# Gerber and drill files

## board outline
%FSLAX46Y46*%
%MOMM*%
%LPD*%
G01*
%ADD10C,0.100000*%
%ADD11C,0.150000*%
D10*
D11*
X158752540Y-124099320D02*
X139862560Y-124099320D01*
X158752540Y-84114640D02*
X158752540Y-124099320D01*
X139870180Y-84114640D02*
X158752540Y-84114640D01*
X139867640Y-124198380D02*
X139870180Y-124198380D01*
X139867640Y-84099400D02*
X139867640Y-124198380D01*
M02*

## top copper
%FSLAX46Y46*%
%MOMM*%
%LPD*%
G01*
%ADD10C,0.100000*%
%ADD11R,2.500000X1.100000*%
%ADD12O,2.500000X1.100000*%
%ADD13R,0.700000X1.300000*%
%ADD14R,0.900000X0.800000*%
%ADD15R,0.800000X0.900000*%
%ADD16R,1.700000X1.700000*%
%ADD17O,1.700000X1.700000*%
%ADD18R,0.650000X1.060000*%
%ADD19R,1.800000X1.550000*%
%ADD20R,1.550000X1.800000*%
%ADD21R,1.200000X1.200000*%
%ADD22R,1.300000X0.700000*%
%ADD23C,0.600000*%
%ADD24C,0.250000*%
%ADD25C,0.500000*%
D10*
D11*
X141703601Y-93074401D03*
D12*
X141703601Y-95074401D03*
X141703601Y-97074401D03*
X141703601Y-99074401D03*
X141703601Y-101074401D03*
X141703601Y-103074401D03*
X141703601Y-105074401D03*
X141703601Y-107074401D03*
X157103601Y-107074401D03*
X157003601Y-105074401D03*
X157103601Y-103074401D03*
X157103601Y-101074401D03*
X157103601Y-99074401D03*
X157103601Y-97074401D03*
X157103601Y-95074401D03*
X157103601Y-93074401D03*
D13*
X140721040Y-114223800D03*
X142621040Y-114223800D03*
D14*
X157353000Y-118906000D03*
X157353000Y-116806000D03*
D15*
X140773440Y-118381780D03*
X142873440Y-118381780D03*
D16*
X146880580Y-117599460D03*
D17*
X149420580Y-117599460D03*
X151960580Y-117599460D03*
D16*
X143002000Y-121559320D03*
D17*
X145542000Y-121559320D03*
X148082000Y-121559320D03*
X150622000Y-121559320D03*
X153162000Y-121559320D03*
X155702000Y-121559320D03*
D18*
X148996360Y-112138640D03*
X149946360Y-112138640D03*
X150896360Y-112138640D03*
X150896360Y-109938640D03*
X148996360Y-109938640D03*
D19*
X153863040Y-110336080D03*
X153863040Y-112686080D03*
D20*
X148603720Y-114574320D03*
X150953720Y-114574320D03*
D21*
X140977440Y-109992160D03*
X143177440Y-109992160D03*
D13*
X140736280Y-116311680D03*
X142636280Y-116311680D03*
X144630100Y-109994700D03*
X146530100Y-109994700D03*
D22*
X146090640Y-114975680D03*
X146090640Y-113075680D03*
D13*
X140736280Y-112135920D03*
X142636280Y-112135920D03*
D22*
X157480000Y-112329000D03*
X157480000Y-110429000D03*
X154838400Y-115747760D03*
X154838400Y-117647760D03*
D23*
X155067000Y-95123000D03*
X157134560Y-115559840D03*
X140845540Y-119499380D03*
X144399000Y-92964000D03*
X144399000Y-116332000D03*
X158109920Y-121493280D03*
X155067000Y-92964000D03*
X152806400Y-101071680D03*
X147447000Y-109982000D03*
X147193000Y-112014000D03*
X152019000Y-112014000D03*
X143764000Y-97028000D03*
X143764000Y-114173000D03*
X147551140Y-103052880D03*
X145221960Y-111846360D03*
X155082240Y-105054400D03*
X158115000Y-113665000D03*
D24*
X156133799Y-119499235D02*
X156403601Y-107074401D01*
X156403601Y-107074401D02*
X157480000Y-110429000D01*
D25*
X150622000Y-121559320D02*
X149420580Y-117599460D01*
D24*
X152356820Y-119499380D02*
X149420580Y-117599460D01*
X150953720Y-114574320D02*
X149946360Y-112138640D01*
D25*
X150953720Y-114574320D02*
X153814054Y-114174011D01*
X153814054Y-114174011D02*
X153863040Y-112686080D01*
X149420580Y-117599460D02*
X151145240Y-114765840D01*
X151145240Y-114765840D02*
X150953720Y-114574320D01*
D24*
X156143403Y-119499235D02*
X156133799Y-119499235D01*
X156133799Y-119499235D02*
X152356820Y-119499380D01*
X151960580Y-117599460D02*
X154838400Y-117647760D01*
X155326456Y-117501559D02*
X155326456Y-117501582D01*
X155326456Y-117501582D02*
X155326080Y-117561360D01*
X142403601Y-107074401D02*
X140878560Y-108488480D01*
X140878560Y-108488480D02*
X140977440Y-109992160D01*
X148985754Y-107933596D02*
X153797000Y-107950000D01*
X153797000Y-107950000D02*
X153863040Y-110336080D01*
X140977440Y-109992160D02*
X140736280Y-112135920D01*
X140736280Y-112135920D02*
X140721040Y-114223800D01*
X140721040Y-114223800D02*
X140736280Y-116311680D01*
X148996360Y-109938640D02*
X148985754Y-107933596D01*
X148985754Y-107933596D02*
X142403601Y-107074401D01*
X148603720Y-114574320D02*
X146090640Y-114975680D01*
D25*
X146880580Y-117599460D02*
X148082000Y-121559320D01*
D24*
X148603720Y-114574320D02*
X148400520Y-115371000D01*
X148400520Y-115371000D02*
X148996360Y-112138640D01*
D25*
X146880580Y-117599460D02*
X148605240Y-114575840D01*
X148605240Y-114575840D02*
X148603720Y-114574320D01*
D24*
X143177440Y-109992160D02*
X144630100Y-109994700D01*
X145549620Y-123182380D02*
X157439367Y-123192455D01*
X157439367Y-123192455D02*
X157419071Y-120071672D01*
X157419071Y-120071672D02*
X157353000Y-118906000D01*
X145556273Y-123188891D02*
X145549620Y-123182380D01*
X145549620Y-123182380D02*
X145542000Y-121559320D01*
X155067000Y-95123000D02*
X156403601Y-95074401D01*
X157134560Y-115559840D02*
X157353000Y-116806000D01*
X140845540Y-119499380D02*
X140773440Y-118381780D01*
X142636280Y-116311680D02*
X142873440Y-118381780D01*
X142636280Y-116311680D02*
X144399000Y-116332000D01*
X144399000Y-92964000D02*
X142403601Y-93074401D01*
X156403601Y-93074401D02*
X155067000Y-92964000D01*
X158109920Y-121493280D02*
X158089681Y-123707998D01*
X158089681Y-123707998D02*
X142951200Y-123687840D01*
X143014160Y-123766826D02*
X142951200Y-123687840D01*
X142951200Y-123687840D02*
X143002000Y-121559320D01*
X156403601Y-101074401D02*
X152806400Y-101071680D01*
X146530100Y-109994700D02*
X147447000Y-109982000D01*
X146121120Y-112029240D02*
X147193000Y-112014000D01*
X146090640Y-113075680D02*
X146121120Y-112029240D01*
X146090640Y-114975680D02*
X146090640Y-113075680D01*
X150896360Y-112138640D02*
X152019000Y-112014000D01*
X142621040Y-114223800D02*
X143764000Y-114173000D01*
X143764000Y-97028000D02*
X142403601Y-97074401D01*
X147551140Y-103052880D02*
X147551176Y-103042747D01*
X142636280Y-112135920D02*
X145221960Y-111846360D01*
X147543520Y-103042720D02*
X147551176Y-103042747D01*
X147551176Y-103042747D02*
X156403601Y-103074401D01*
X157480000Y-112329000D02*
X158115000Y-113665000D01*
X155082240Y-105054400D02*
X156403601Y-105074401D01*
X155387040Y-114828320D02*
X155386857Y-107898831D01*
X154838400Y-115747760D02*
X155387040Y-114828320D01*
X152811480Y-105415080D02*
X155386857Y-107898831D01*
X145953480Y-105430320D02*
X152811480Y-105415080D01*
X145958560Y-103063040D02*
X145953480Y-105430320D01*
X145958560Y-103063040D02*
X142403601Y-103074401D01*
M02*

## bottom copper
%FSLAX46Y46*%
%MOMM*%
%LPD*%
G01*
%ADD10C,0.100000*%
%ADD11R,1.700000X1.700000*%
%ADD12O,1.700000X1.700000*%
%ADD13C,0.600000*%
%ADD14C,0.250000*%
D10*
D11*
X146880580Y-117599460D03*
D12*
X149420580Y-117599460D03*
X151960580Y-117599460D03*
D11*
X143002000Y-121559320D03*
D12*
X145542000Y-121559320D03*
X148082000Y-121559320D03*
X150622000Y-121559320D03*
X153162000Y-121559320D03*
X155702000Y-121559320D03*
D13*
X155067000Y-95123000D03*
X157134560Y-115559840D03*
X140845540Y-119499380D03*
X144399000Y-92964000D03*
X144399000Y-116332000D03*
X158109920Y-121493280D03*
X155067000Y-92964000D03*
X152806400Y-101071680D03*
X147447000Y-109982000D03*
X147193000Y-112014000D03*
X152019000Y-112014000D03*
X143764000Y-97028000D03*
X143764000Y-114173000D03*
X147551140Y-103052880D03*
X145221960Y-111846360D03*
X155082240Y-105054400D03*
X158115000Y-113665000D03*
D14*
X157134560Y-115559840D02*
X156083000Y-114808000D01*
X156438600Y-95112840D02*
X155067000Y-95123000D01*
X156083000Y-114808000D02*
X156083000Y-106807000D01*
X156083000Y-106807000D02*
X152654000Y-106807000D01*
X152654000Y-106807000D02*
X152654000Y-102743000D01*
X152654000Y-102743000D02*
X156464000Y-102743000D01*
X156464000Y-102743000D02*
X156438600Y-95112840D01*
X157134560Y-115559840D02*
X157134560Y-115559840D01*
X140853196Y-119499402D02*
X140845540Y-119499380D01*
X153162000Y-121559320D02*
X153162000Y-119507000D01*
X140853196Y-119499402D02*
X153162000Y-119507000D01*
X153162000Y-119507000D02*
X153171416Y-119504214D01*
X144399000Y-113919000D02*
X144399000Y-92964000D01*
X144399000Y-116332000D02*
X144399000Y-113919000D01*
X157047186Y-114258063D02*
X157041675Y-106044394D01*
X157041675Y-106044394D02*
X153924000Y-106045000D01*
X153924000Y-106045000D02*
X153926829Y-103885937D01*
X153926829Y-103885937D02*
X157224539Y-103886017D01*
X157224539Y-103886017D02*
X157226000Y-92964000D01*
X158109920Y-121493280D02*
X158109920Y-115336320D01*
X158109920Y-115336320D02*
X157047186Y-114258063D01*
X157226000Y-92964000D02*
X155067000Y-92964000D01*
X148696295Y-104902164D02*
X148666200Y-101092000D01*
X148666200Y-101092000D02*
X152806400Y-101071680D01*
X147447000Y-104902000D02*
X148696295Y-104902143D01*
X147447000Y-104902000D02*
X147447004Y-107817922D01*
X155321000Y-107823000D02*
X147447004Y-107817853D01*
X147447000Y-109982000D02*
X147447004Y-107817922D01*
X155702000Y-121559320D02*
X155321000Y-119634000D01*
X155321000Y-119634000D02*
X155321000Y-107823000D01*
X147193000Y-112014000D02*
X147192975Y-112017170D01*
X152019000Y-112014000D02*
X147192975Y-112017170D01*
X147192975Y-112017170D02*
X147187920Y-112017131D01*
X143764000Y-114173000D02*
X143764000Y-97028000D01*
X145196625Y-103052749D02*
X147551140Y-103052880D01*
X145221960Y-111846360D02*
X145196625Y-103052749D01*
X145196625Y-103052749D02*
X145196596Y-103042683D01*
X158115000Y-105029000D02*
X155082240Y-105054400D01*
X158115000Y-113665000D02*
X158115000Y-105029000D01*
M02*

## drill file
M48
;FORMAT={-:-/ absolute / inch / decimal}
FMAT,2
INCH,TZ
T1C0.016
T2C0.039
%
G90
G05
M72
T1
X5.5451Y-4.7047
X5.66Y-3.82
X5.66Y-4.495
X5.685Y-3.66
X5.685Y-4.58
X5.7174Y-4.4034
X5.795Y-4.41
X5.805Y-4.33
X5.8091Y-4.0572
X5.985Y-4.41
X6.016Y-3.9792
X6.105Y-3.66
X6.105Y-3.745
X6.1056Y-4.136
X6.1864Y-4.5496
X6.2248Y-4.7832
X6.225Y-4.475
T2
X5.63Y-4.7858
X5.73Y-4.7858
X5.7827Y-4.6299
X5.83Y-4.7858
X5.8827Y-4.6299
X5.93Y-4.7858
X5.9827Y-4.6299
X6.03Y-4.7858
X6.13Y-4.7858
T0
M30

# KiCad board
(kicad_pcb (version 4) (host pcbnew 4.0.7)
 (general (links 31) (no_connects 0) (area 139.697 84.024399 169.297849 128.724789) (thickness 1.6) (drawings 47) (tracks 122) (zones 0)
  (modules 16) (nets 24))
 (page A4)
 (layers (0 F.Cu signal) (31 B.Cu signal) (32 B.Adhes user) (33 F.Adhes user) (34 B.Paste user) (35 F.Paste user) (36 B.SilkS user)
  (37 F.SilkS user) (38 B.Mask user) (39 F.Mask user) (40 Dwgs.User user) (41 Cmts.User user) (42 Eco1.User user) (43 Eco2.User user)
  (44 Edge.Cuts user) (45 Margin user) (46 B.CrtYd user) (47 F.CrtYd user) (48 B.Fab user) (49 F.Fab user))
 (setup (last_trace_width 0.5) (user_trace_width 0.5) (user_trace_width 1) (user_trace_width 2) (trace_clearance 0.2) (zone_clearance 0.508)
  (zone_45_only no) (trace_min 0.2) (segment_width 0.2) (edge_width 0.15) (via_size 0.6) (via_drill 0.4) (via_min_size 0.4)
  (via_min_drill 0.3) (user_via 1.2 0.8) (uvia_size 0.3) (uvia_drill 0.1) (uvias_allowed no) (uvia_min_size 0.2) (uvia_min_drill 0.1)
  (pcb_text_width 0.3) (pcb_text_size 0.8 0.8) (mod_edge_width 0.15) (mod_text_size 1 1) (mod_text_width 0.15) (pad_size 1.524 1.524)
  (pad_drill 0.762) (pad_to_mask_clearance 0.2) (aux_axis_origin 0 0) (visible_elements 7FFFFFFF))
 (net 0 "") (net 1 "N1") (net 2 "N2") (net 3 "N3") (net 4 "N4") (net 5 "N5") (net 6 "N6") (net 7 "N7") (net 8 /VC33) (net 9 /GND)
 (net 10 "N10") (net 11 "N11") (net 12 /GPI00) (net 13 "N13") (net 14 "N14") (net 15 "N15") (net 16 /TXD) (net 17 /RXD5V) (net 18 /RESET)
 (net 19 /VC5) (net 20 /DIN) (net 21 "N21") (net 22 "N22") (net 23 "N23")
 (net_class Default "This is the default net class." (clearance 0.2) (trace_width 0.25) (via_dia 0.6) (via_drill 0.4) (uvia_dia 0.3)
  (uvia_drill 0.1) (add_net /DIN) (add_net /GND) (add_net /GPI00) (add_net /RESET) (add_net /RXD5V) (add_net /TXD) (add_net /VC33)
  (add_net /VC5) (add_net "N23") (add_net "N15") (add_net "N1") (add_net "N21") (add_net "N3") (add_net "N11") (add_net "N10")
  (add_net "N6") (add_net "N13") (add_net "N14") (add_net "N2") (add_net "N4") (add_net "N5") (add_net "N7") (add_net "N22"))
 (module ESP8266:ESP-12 (layer F.Cu) (at 142.403601 93.074401)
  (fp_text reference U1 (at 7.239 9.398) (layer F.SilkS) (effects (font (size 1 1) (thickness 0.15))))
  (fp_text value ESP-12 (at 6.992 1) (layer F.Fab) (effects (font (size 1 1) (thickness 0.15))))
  (pad 1 smd rect (at 0 0) (size 2.5 1.1) (drill (offset -0.7 0)) (layers F.Cu F.Paste F.Mask) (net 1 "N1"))
  (pad 2 smd oval (at 0 2) (size 2.5 1.1) (drill (offset -0.7 0)) (layers F.Cu F.Paste F.Mask) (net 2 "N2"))
  (pad 3 smd oval (at 0 4) (size 2.5 1.1) (drill (offset -0.7 0)) (layers F.Cu F.Paste F.Mask) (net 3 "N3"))
  (pad 4 smd oval (at 0 6) (size 2.5 1.1) (drill (offset -0.7 0)) (layers F.Cu F.Paste F.Mask) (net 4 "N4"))
  (pad 5 smd oval (at 0 8) (size 2.5 1.1) (drill (offset -0.7 0)) (layers F.Cu F.Paste F.Mask) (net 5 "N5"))
  (pad 6 smd oval (at 0 10) (size 2.5 1.1) (drill (offset -0.7 0)) (layers F.Cu F.Paste F.Mask) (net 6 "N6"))
  (pad 7 smd oval (at 0 12) (size 2.5 1.1) (drill (offset -0.7 0)) (layers F.Cu F.Paste F.Mask) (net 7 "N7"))
  (pad 8 smd oval (at 0 14) (size 2.5 1.1) (drill (offset -0.7 0)) (layers F.Cu F.Paste F.Mask) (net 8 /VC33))
  (pad 9 smd oval (at 14 14) (size 2.5 1.1) (drill (offset 0.7 0)) (layers F.Cu F.Paste F.Mask) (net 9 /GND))
  (pad 10 smd oval (at 14 12) (size 2.5 1.1) (drill (offset 0.6 0)) (layers F.Cu F.Paste F.Mask) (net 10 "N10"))
  (pad 11 smd oval (at 14 10) (size 2.5 1.1) (drill (offset 0.7 0)) (layers F.Cu F.Paste F.Mask) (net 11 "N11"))
  (pad 12 smd oval (at 14 8) (size 2.5 1.1) (drill (offset 0.7 0)) (layers F.Cu F.Paste F.Mask) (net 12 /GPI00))
  (pad 13 smd oval (at 14 6) (size 2.5 1.1) (drill (offset 0.7 0)) (layers F.Cu F.Paste F.Mask) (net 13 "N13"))
  (pad 14 smd oval (at 14 4) (size 2.5 1.1) (drill (offset 0.7 0)) (layers F.Cu F.Paste F.Mask) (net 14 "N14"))
  (pad 15 smd oval (at 14 2) (size 2.5 1.1) (drill (offset 0.7 0)) (layers F.Cu F.Paste F.Mask) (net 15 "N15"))
  (pad 16 smd oval (at 14 0) (size 2.5 1.1) (drill (offset 0.7 0)) (layers F.Cu F.Paste F.Mask) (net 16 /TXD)))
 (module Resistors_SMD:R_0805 (layer F.Cu) (at 141.67104 114.2238)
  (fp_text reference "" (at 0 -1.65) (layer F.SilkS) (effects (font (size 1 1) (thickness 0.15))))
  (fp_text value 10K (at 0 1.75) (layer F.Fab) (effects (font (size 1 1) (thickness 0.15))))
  (pad 1 smd rect (at -0.95 0) (size 0.7 1.3) (layers F.Cu F.Paste F.Mask) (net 8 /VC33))
  (pad 2 smd rect (at 0.95 0) (size 0.7 1.3) (layers F.Cu F.Paste F.Mask) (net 3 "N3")))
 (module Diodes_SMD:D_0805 (layer F.Cu) (at 157.353 117.856 90)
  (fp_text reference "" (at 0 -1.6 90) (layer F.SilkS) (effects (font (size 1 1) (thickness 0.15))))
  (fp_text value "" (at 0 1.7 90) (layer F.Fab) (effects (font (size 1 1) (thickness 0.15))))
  (pad 1 smd rect (at -1.05 0 90) (size 0.8 0.9) (layers F.Cu F.Paste F.Mask) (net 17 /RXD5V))
  (pad 2 smd rect (at 1.05 0 90) (size 0.8 0.9) (layers F.Cu F.Paste F.Mask) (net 15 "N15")))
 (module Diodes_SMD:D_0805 (layer F.Cu) (at 141.82344 118.38178)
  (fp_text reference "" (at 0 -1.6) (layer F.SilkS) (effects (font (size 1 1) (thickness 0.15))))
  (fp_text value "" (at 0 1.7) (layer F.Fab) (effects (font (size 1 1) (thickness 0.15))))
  (pad 1 smd rect (at -1.05 0) (size 0.8 0.9) (layers F.Cu F.Paste F.Mask) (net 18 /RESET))
  (pad 2 smd rect (at 1.05 0) (size 0.8 0.9) (layers F.Cu F.Paste F.Mask) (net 1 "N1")))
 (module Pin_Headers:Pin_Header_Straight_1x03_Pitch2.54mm (layer F.Cu) (at 146.88058 117.59946 90)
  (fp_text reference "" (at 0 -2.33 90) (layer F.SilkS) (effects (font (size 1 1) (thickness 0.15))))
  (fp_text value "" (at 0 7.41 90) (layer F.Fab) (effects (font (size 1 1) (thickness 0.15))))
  (pad 1 thru_hole rect (at 0 0 90) (size 1.7 1.7) (drill 1) (layers *.Cu *.Mask) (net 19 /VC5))
  (pad 2 thru_hole oval (at 0 2.54 90) (size 1.7 1.7) (drill 1) (layers *.Cu *.Mask) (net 9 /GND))
  (pad 3 thru_hole oval (at 0 5.08 90) (size 1.7 1.7) (drill 1) (layers *.Cu *.Mask) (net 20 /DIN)))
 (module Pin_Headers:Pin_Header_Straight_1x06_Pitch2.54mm (layer F.Cu) (at 143.002 121.55932 90)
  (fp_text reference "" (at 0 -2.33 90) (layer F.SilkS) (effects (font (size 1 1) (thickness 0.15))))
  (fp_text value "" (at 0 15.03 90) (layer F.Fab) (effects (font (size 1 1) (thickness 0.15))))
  (pad 1 thru_hole rect (at 0 0 90) (size 1.7 1.7) (drill 1) (layers *.Cu *.Mask) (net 16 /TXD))
  (pad 2 thru_hole oval (at 0 2.54 90) (size 1.7 1.7) (drill 1) (layers *.Cu *.Mask) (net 17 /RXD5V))
  (pad 3 thru_hole oval (at 0 5.08 90) (size 1.7 1.7) (drill 1) (layers *.Cu *.Mask) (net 19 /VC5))
  (pad 4 thru_hole oval (at 0 7.62 90) (size 1.7 1.7) (drill 1) (layers *.Cu *.Mask) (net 9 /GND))
  (pad 5 thru_hole oval (at 0 10.16 90) (size 1.7 1.7) (drill 1) (layers *.Cu *.Mask) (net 18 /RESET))
  (pad 6 thru_hole oval (at 0 12.7 90) (size 1.7 1.7) (drill 1) (layers *.Cu *.Mask) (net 12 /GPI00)))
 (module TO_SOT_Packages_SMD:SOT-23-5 (layer F.Cu) (at 149.94636 111.03864 90)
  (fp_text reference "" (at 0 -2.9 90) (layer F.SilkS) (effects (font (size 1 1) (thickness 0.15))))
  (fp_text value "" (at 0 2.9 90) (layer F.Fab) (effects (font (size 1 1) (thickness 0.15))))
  (pad 1 smd rect (at -1.1 -0.95 90) (size 1.06 0.65) (layers F.Cu F.Paste F.Mask) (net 19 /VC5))
  (pad 2 smd rect (at -1.1 0 90) (size 1.06 0.65) (layers F.Cu F.Paste F.Mask) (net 9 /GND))
  (pad 3 smd rect (at -1.1 0.95 90) (size 1.06 0.65) (layers F.Cu F.Paste F.Mask) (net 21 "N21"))
  (pad 4 smd rect (at 1.1 0.95 90) (size 1.06 0.65) (layers F.Cu F.Paste F.Mask) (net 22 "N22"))
  (pad 5 smd rect (at 1.1 -0.95 90) (size 1.06 0.65) (layers F.Cu F.Paste F.Mask) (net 8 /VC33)))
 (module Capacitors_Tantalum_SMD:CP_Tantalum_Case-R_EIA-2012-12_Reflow (layer F.Cu) (at 153.86304 111.51108 270)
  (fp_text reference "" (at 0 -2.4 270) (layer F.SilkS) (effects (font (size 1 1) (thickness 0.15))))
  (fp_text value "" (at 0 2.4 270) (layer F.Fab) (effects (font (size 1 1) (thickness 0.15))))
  (pad 1 smd rect (at -1.175 0 270) (size 1.55 1.8) (layers F.Cu F.Paste F.Mask) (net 8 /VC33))
  (pad 2 smd rect (at 1.175 0 270) (size 1.55 1.8) (layers F.Cu F.Paste F.Mask) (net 9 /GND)))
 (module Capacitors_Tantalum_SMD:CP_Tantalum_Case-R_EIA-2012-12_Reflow (layer F.Cu) (at 149.77872 114.57432)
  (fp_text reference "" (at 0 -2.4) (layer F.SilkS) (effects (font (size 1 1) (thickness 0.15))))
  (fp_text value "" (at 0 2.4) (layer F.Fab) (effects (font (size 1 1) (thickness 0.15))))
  (pad 1 smd rect (at -1.175 0) (size 1.55 1.8) (layers F.Cu F.Paste F.Mask) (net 19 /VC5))
  (pad 2 smd rect (at 1.175 0) (size 1.55 1.8) (layers F.Cu F.Paste F.Mask) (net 9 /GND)))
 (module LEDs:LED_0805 (layer F.Cu) (at 142.07744 109.99216 180)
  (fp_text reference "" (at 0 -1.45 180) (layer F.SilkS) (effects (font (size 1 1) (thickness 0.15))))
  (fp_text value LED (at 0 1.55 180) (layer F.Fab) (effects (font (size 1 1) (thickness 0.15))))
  (pad 2 smd rect (at 1.1 0) (size 1.2 1.2) (layers F.Cu F.Paste F.Mask) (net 8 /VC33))
  (pad 1 smd rect (at -1.1 0) (size 1.2 1.2) (layers F.Cu F.Paste F.Mask) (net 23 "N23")))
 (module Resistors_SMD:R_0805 (layer F.Cu) (at 141.68628 116.31168)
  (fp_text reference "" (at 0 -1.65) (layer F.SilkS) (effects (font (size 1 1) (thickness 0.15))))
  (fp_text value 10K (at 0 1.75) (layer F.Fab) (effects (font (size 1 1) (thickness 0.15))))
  (pad 1 smd rect (at -0.95 0) (size 0.7 1.3) (layers F.Cu F.Paste F.Mask) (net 8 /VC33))
  (pad 2 smd rect (at 0.95 0) (size 0.7 1.3) (layers F.Cu F.Paste F.Mask) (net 1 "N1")))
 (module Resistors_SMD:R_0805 (layer F.Cu) (at 145.5801 109.9947)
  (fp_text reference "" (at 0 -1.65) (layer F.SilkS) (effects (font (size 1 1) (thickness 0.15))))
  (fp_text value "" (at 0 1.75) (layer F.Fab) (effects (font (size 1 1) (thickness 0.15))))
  (pad 1 smd rect (at -0.95 0) (size 0.7 1.3) (layers F.Cu F.Paste F.Mask) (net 23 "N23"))
  (pad 2 smd rect (at 0.95 0) (size 0.7 1.3) (layers F.Cu F.Paste F.Mask) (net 12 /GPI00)))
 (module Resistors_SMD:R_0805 (layer F.Cu) (at 146.09064 114.02568 90)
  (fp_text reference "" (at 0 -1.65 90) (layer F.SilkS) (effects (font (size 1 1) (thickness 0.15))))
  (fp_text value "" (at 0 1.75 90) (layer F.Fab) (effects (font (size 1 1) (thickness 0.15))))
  (pad 1 smd rect (at -0.95 0 90) (size 0.7 1.3) (layers F.Cu F.Paste F.Mask) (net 19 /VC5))
  (pad 2 smd rect (at 0.95 0 90) (size 0.7 1.3) (layers F.Cu F.Paste F.Mask) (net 21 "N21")))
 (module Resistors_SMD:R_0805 (layer F.Cu) (at 141.68628 112.13592)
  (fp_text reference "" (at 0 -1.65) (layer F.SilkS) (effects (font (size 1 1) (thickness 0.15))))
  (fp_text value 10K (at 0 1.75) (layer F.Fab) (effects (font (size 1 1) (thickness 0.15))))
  (pad 1 smd rect (at -0.95 0) (size 0.7 1.3) (layers F.Cu F.Paste F.Mask) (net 8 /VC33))
  (pad 2 smd rect (at 0.95 0) (size 0.7 1.3) (layers F.Cu F.Paste F.Mask) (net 11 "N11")))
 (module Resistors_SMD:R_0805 (layer F.Cu) (at 157.48 111.379 90)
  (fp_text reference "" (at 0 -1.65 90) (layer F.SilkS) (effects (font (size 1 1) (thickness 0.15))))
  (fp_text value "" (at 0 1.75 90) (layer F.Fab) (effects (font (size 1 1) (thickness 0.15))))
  (pad 1 smd rect (at -0.95 0 90) (size 0.7 1.3) (layers F.Cu F.Paste F.Mask) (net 10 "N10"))
  (pad 2 smd rect (at 0.95 0 90) (size 0.7 1.3) (layers F.Cu F.Paste F.Mask) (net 9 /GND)))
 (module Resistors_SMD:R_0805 (layer F.Cu) (at 154.8384 116.69776 270)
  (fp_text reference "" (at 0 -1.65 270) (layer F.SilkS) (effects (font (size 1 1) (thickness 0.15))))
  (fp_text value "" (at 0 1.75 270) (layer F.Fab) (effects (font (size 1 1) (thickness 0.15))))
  (pad 1 smd rect (at -0.95 0 270) (size 0.7 1.3) (layers F.Cu F.Paste F.Mask) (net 6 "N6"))
  (pad 2 smd rect (at 0.95 0 270) (size 0.7 1.3) (layers F.Cu F.Paste F.Mask) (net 20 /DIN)))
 (gr_line (start 158.75254 124.09932) (end 139.86256 124.09932) (angle 90) (layer Edge.Cuts) (width 0.15))
 (gr_line (start 158.75254 84.11464) (end 158.75254 124.09932) (angle 90) (layer Edge.Cuts) (width 0.15))
 (gr_line (start 139.87018 84.11464) (end 158.75254 84.11464) (angle 90) (layer Edge.Cuts) (width 0.15))
 (gr_line (start 139.86764 124.19838) (end 139.87018 124.19838) (angle 90) (layer Edge.Cuts) (width 0.15))
 (gr_line (start 139.86764 84.0994) (end 139.86764 124.19838) (angle 90) (layer Edge.Cuts) (width 0.15))
 (segment (start 156.133799 119.499235) (end 156.403601 107.074401) (width 0.25) (layer F.Cu) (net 9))
 (segment (start 156.403601 107.074401) (end 157.48 110.429) (width 0.25) (layer F.Cu) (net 9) (status 20))
 (segment (start 150.622 121.55932) (end 149.42058 117.59946) (width 0.5) (layer F.Cu) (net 9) (status 20))
 (segment (start 152.35682 119.49938) (end 149.42058 117.59946) (width 0.25) (layer F.Cu) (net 9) (status 20))
 (segment (start 150.95372 114.57432) (end 149.94636 112.13864) (width 0.25) (layer F.Cu) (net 9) (status 10))
 (segment (start 150.95372 114.57432) (end 153.814054 114.174011) (width 0.5) (layer F.Cu) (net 9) (status 10))
 (segment (start 153.814054 114.174011) (end 153.86304 112.68608) (width 0.5) (layer F.Cu) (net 9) (status 10))
 (segment (start 149.42058 117.59946) (end 151.14524 114.76584) (width 0.5) (layer F.Cu) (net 9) (status 20))
 (segment (start 151.14524 114.76584) (end 150.95372 114.57432) (width 0.5) (layer F.Cu) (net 9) (status 30))
 (segment (start 156.143403 119.499235) (end 156.133799 119.499235) (width 0.25) (layer F.Cu) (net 9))
 (segment (start 156.133799 119.499235) (end 152.35682 119.49938) (width 0.25) (layer F.Cu) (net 9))
 (segment (start 151.96058 117.59946) (end 154.8384 117.64776) (width 0.25) (layer F.Cu) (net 20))
 (segment (start 155.326456 117.501559) (end 155.326456 117.501582) (width 0.25) (layer F.Cu) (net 20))
 (segment (start 155.326456 117.501582) (end 155.32608 117.56136) (width 0.25) (layer F.Cu) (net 20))
 (segment (start 142.403601 107.074401) (end 140.87856 108.48848) (width 0.25) (layer F.Cu) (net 8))
 (segment (start 140.87856 108.48848) (end 140.97744 109.99216) (width 0.25) (layer F.Cu) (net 8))
 (segment (start 148.985754 107.933596) (end 153.797 107.95) (width 0.25) (layer F.Cu) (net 8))
 (segment (start 153.797 107.95) (end 153.86304 110.33608) (width 0.25) (layer F.Cu) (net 8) (status 20))
 (segment (start 140.97744 109.99216) (end 140.73628 112.13592) (width 0.25) (layer F.Cu) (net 8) (status 20))
 (segment (start 140.73628 112.13592) (end 140.72104 114.2238) (width 0.25) (layer F.Cu) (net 8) (status 20))
 (segment (start 140.72104 114.2238) (end 140.73628 116.31168) (width 0.25) (layer F.Cu) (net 8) (status 20))
 (segment (start 148.99636 109.93864) (end 148.985754 107.933596) (width 0.25) (layer F.Cu) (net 8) (status 10))
 (segment (start 148.985754 107.933596) (end 142.403601 107.074401) (width 0.25) (layer F.Cu) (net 8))
 (segment (start 148.60372 114.57432) (end 146.09064 114.97568) (width 0.25) (layer F.Cu) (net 19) (status 10))
 (segment (start 146.88058 117.59946) (end 148.082 121.55932) (width 0.5) (layer F.Cu) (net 19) (status 10))
 (segment (start 148.60372 114.57432) (end 148.40052 115.371) (width 0.25) (layer F.Cu) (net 19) (status 30))
 (segment (start 148.40052 115.371) (end 148.99636 112.13864) (width 0.25) (layer F.Cu) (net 19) (status 10))
 (segment (start 146.88058 117.59946) (end 148.60524 114.57584) (width 0.5) (layer F.Cu) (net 19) (status 20))
 (segment (start 148.60524 114.57584) (end 148.60372 114.57432) (width 0.5) (layer F.Cu) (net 19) (status 30))
 (segment (start 143.17744 109.99216) (end 144.6301 109.9947) (width 0.25) (layer F.Cu) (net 23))
 (segment (start 145.54962 123.18238) (end 157.439367 123.192455) (width 0.25) (layer F.Cu) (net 17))
 (segment (start 157.439367 123.192455) (end 157.419071 120.071672) (width 0.25) (layer F.Cu) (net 17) (status 20))
 (segment (start 157.419071 120.071672) (end 157.353 118.906) (width 0.25) (layer F.Cu) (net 17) (status 20))
 (segment (start 145.556273 123.188891) (end 145.54962 123.18238) (width 0.25) (layer F.Cu) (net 17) (status 20))
 (segment (start 145.54962 123.18238) (end 145.542 121.55932) (width 0.25) (layer F.Cu) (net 17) (status 20))
 (segment (start 157.13456 115.55984) (end 156.083 114.808) (width 0.25) (layer B.Cu) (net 15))
 (via (at 155.067 95.123) (size 0.6) (drill 0.4) (layers F.Cu B.Cu) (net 15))
 (segment (start 155.067 95.123) (end 156.403601 95.074401) (width 0.25) (layer F.Cu) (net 15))
 (segment (start 156.4386 95.11284) (end 155.067 95.123) (width 0.25) (layer B.Cu) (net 15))
 (segment (start 156.083 114.808) (end 156.083 106.807) (width 0.25) (layer B.Cu) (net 15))
 (segment (start 156.083 106.807) (end 152.654 106.807) (width 0.25) (layer B.Cu) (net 15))
 (segment (start 152.654 106.807) (end 152.654 102.743) (width 0.25) (layer B.Cu) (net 15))
 (segment (start 152.654 102.743) (end 156.464 102.743) (width 0.25) (layer B.Cu) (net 15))
 (segment (start 156.464 102.743) (end 156.4386 95.11284) (width 0.25) (layer B.Cu) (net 15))
 (segment (start 157.13456 115.55984) (end 157.353 116.806) (width 0.25) (layer F.Cu) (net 15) (status 20))
 (via (at 157.13456 115.55984) (size 0.6) (drill 0.4) (layers F.Cu B.Cu) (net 15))
 (segment (start 157.13456 115.55984) (end 157.13456 115.55984) (width 0.25) (layer B.Cu) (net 15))
 (segment (start 140.853196 119.499402) (end 140.84554 119.49938) (width 0.25) (layer B.Cu) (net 18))
 (via (at 140.84554 119.49938) (size 0.6) (drill 0.4) (layers F.Cu B.Cu) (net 18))
 (segment (start 140.84554 119.49938) (end 140.77344 118.38178) (width 0.25) (layer F.Cu) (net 18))
 (segment (start 153.162 121.55932) (end 153.162 119.507) (width 0.25) (layer B.Cu) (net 18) (status 10))
 (segment (start 140.853196 119.499402) (end 153.162 119.507) (width 0.25) (layer B.Cu) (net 18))
 (segment (start 153.162 119.507) (end 153.171416 119.504214) (width 0.25) (layer B.Cu) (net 18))
 (segment (start 142.63628 116.31168) (end 142.87344 118.38178) (width 0.25) (layer F.Cu) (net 1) (status 10))
 (segment (start 142.63628 116.31168) (end 144.399 116.332) (width 0.25) (layer F.Cu) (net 1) (status 10))
 (segment (start 144.399 92.964) (end 142.403601 93.074401) (width 0.25) (layer F.Cu) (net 1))
 (via (at 144.399 92.964) (size 0.6) (drill 0.4) (layers F.Cu B.Cu) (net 1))
 (segment (start 144.399 113.919) (end 144.399 92.964) (width 0.25) (layer B.Cu) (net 1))
 (segment (start 144.399 116.332) (end 144.399 113.919) (width 0.25) (layer B.Cu) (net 1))
 (via (at 144.399 116.332) (size 0.6) (drill 0.4) (layers F.Cu B.Cu) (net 1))
 (segment (start 157.047186 114.258063) (end 157.041675 106.044394) (width 0.25) (layer B.Cu) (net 16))
 (segment (start 157.041675 106.044394) (end 153.924 106.045) (width 0.25) (layer B.Cu) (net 16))
 (segment (start 153.924 106.045) (end 153.926829 103.885937) (width 0.25) (layer B.Cu) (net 16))
 (segment (start 153.926829 103.885937) (end 157.224539 103.886017) (width 0.25) (layer B.Cu) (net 16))
 (segment (start 157.224539 103.886017) (end 157.226 92.964) (width 0.25) (layer B.Cu) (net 16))
 (via (at 158.10992 121.49328) (size 0.6) (drill 0.4) (layers F.Cu B.Cu) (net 16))
 (segment (start 158.10992 121.49328) (end 158.10992 115.33632) (width 0.25) (layer B.Cu) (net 16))
 (via (at 155.067 92.964) (size 0.6) (drill 0.4) (layers F.Cu B.Cu) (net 16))
 (segment (start 156.403601 93.074401) (end 155.067 92.964) (width 0.25) (layer F.Cu) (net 16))
 (segment (start 158.10992 121.49328) (end 158.089681 123.707998) (width 0.25) (layer F.Cu) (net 16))
 (segment (start 158.089681 123.707998) (end 142.9512 123.68784) (width 0.25) (layer F.Cu) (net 16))
 (segment (start 158.10992 115.33632) (end 157.047186 114.258063) (width 0.25) (layer B.Cu) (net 16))
 (segment (start 157.226 92.964) (end 155.067 92.964) (width 0.25) (layer B.Cu) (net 16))
 (segment (start 143.01416 123.766826) (end 142.9512 123.68784) (width 0.25) (layer F.Cu) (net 16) (status 20))
 (segment (start 142.9512 123.68784) (end 143.002 121.55932) (width 0.25) (layer F.Cu) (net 16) (status 20))
 (segment (start 148.696295 104.902164) (end 148.6662 101.092) (width 0.25) (layer B.Cu) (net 12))
 (segment (start 148.6662 101.092) (end 152.8064 101.07168) (width 0.25) (layer B.Cu) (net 12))
 (segment (start 156.403601 101.074401) (end 152.8064 101.07168) (width 0.25) (layer F.Cu) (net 12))
 (via (at 152.8064 101.07168) (size 0.6) (drill 0.4) (layers F.Cu B.Cu) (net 12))
 (segment (start 147.447 104.902) (end 148.696295 104.902143) (width 0.25) (layer B.Cu) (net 12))
 (segment (start 147.447 104.902) (end 147.447004 107.817922) (width 0.25) (layer B.Cu) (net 12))
 (segment (start 155.321 107.823) (end 147.447004 107.817853) (width 0.25) (layer B.Cu) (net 12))
 (segment (start 146.5301 109.9947) (end 147.447 109.982) (width 0.25) (layer F.Cu) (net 12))
 (via (at 147.447 109.982) (size 0.6) (drill 0.4) (layers F.Cu B.Cu) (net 12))
 (segment (start 147.447 109.982) (end 147.447004 107.817922) (width 0.25) (layer B.Cu) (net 12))
 (segment (start 155.702 121.55932) (end 155.321 119.634) (width 0.25) (layer B.Cu) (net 12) (status 10))
 (segment (start 155.321 119.634) (end 155.321 107.823) (width 0.25) (layer B.Cu) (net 12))
 (segment (start 146.12112 112.02924) (end 147.193 112.014) (width 0.25) (layer F.Cu) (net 21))
 (segment (start 146.09064 113.07568) (end 146.12112 112.02924) (width 0.25) (layer F.Cu) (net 21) (status 20))
 (segment (start 147.193 112.014) (end 147.192975 112.01717) (width 0.25) (layer B.Cu) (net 21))
 (via (at 147.193 112.014) (size 0.6) (drill 0.4) (layers F.Cu B.Cu) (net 21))
 (segment (start 146.09064 114.97568) (end 146.09064 113.07568) (width 0.25) (layer F.Cu) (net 21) (status 30))
 (segment (start 150.89636 112.13864) (end 152.019 112.014) (width 0.25) (layer F.Cu) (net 21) (status 10))
 (segment (start 152.019 112.014) (end 147.192975 112.01717) (width 0.25) (layer B.Cu) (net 21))
 (via (at 152.019 112.014) (size 0.6) (drill 0.4) (layers F.Cu B.Cu) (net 21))
 (segment (start 147.192975 112.01717) (end 147.18792 112.017131) (width 0.25) (layer B.Cu) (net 21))
 (segment (start 142.62104 114.2238) (end 143.764 114.173) (width 0.25) (layer F.Cu) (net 3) (status 10))
 (segment (start 143.764 97.028) (end 142.403601 97.074401) (width 0.25) (layer F.Cu) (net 3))
 (via (at 143.764 97.028) (size 0.6) (drill 0.4) (layers F.Cu B.Cu) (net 3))
 (segment (start 143.764 114.173) (end 143.764 97.028) (width 0.25) (layer B.Cu) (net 3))
 (via (at 143.764 114.173) (size 0.6) (drill 0.4) (layers F.Cu B.Cu) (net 3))
 (segment (start 145.196625 103.052749) (end 147.55114 103.05288) (width 0.25) (layer B.Cu) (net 11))
 (segment (start 147.55114 103.05288) (end 147.551176 103.042747) (width 0.25) (layer F.Cu) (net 11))
 (via (at 147.55114 103.05288) (size 0.6) (drill 0.4) (layers F.Cu B.Cu) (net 11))
 (segment (start 142.63628 112.13592) (end 145.22196 111.84636) (width 0.25) (layer F.Cu) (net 11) (status 10))
 (via (at 145.22196 111.84636) (size 0.6) (drill 0.4) (layers F.Cu B.Cu) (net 11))
 (segment (start 145.22196 111.84636) (end 145.196625 103.052749) (width 0.25) (layer B.Cu) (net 11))
 (segment (start 145.196625 103.052749) (end 145.196596 103.042683) (width 0.25) (layer B.Cu) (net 11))
 (segment (start 147.54352 103.04272) (end 147.551176 103.042747) (width 0.25) (layer F.Cu) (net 11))
 (segment (start 147.551176 103.042747) (end 156.403601 103.074401) (width 0.25) (layer F.Cu) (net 11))
 (segment (start 157.48 112.329) (end 158.115 113.665) (width 0.25) (layer F.Cu) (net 10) (status 10))
 (segment (start 155.08224 105.0544) (end 156.403601 105.074401) (width 0.25) (layer F.Cu) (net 10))
 (via (at 155.08224 105.0544) (size 0.6) (drill 0.4) (layers F.Cu B.Cu) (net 10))
 (segment (start 158.115 105.029) (end 155.08224 105.0544) (width 0.25) (layer B.Cu) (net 10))
 (segment (start 158.115 113.665) (end 158.115 105.029) (width 0.25) (layer B.Cu) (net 10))
 (via (at 158.115 113.665) (size 0.6) (drill 0.4) (layers F.Cu B.Cu) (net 10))
 (segment (start 155.38704 114.82832) (end 155.386857 107.898831) (width 0.25) (layer F.Cu) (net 6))
 (segment (start 154.8384 115.74776) (end 155.38704 114.82832) (width 0.25) (layer F.Cu) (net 6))
 (segment (start 152.81148 105.41508) (end 155.386857 107.898831) (width 0.25) (layer F.Cu) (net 6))
 (segment (start 145.95348 105.43032) (end 152.81148 105.41508) (width 0.25) (layer F.Cu) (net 6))
 (segment (start 145.95856 103.06304) (end 145.95348 105.43032) (width 0.25) (layer F.Cu) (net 6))
 (segment (start 145.95856 103.06304) (end 142.403601 103.074401) (width 0.25) (layer F.Cu) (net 6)))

